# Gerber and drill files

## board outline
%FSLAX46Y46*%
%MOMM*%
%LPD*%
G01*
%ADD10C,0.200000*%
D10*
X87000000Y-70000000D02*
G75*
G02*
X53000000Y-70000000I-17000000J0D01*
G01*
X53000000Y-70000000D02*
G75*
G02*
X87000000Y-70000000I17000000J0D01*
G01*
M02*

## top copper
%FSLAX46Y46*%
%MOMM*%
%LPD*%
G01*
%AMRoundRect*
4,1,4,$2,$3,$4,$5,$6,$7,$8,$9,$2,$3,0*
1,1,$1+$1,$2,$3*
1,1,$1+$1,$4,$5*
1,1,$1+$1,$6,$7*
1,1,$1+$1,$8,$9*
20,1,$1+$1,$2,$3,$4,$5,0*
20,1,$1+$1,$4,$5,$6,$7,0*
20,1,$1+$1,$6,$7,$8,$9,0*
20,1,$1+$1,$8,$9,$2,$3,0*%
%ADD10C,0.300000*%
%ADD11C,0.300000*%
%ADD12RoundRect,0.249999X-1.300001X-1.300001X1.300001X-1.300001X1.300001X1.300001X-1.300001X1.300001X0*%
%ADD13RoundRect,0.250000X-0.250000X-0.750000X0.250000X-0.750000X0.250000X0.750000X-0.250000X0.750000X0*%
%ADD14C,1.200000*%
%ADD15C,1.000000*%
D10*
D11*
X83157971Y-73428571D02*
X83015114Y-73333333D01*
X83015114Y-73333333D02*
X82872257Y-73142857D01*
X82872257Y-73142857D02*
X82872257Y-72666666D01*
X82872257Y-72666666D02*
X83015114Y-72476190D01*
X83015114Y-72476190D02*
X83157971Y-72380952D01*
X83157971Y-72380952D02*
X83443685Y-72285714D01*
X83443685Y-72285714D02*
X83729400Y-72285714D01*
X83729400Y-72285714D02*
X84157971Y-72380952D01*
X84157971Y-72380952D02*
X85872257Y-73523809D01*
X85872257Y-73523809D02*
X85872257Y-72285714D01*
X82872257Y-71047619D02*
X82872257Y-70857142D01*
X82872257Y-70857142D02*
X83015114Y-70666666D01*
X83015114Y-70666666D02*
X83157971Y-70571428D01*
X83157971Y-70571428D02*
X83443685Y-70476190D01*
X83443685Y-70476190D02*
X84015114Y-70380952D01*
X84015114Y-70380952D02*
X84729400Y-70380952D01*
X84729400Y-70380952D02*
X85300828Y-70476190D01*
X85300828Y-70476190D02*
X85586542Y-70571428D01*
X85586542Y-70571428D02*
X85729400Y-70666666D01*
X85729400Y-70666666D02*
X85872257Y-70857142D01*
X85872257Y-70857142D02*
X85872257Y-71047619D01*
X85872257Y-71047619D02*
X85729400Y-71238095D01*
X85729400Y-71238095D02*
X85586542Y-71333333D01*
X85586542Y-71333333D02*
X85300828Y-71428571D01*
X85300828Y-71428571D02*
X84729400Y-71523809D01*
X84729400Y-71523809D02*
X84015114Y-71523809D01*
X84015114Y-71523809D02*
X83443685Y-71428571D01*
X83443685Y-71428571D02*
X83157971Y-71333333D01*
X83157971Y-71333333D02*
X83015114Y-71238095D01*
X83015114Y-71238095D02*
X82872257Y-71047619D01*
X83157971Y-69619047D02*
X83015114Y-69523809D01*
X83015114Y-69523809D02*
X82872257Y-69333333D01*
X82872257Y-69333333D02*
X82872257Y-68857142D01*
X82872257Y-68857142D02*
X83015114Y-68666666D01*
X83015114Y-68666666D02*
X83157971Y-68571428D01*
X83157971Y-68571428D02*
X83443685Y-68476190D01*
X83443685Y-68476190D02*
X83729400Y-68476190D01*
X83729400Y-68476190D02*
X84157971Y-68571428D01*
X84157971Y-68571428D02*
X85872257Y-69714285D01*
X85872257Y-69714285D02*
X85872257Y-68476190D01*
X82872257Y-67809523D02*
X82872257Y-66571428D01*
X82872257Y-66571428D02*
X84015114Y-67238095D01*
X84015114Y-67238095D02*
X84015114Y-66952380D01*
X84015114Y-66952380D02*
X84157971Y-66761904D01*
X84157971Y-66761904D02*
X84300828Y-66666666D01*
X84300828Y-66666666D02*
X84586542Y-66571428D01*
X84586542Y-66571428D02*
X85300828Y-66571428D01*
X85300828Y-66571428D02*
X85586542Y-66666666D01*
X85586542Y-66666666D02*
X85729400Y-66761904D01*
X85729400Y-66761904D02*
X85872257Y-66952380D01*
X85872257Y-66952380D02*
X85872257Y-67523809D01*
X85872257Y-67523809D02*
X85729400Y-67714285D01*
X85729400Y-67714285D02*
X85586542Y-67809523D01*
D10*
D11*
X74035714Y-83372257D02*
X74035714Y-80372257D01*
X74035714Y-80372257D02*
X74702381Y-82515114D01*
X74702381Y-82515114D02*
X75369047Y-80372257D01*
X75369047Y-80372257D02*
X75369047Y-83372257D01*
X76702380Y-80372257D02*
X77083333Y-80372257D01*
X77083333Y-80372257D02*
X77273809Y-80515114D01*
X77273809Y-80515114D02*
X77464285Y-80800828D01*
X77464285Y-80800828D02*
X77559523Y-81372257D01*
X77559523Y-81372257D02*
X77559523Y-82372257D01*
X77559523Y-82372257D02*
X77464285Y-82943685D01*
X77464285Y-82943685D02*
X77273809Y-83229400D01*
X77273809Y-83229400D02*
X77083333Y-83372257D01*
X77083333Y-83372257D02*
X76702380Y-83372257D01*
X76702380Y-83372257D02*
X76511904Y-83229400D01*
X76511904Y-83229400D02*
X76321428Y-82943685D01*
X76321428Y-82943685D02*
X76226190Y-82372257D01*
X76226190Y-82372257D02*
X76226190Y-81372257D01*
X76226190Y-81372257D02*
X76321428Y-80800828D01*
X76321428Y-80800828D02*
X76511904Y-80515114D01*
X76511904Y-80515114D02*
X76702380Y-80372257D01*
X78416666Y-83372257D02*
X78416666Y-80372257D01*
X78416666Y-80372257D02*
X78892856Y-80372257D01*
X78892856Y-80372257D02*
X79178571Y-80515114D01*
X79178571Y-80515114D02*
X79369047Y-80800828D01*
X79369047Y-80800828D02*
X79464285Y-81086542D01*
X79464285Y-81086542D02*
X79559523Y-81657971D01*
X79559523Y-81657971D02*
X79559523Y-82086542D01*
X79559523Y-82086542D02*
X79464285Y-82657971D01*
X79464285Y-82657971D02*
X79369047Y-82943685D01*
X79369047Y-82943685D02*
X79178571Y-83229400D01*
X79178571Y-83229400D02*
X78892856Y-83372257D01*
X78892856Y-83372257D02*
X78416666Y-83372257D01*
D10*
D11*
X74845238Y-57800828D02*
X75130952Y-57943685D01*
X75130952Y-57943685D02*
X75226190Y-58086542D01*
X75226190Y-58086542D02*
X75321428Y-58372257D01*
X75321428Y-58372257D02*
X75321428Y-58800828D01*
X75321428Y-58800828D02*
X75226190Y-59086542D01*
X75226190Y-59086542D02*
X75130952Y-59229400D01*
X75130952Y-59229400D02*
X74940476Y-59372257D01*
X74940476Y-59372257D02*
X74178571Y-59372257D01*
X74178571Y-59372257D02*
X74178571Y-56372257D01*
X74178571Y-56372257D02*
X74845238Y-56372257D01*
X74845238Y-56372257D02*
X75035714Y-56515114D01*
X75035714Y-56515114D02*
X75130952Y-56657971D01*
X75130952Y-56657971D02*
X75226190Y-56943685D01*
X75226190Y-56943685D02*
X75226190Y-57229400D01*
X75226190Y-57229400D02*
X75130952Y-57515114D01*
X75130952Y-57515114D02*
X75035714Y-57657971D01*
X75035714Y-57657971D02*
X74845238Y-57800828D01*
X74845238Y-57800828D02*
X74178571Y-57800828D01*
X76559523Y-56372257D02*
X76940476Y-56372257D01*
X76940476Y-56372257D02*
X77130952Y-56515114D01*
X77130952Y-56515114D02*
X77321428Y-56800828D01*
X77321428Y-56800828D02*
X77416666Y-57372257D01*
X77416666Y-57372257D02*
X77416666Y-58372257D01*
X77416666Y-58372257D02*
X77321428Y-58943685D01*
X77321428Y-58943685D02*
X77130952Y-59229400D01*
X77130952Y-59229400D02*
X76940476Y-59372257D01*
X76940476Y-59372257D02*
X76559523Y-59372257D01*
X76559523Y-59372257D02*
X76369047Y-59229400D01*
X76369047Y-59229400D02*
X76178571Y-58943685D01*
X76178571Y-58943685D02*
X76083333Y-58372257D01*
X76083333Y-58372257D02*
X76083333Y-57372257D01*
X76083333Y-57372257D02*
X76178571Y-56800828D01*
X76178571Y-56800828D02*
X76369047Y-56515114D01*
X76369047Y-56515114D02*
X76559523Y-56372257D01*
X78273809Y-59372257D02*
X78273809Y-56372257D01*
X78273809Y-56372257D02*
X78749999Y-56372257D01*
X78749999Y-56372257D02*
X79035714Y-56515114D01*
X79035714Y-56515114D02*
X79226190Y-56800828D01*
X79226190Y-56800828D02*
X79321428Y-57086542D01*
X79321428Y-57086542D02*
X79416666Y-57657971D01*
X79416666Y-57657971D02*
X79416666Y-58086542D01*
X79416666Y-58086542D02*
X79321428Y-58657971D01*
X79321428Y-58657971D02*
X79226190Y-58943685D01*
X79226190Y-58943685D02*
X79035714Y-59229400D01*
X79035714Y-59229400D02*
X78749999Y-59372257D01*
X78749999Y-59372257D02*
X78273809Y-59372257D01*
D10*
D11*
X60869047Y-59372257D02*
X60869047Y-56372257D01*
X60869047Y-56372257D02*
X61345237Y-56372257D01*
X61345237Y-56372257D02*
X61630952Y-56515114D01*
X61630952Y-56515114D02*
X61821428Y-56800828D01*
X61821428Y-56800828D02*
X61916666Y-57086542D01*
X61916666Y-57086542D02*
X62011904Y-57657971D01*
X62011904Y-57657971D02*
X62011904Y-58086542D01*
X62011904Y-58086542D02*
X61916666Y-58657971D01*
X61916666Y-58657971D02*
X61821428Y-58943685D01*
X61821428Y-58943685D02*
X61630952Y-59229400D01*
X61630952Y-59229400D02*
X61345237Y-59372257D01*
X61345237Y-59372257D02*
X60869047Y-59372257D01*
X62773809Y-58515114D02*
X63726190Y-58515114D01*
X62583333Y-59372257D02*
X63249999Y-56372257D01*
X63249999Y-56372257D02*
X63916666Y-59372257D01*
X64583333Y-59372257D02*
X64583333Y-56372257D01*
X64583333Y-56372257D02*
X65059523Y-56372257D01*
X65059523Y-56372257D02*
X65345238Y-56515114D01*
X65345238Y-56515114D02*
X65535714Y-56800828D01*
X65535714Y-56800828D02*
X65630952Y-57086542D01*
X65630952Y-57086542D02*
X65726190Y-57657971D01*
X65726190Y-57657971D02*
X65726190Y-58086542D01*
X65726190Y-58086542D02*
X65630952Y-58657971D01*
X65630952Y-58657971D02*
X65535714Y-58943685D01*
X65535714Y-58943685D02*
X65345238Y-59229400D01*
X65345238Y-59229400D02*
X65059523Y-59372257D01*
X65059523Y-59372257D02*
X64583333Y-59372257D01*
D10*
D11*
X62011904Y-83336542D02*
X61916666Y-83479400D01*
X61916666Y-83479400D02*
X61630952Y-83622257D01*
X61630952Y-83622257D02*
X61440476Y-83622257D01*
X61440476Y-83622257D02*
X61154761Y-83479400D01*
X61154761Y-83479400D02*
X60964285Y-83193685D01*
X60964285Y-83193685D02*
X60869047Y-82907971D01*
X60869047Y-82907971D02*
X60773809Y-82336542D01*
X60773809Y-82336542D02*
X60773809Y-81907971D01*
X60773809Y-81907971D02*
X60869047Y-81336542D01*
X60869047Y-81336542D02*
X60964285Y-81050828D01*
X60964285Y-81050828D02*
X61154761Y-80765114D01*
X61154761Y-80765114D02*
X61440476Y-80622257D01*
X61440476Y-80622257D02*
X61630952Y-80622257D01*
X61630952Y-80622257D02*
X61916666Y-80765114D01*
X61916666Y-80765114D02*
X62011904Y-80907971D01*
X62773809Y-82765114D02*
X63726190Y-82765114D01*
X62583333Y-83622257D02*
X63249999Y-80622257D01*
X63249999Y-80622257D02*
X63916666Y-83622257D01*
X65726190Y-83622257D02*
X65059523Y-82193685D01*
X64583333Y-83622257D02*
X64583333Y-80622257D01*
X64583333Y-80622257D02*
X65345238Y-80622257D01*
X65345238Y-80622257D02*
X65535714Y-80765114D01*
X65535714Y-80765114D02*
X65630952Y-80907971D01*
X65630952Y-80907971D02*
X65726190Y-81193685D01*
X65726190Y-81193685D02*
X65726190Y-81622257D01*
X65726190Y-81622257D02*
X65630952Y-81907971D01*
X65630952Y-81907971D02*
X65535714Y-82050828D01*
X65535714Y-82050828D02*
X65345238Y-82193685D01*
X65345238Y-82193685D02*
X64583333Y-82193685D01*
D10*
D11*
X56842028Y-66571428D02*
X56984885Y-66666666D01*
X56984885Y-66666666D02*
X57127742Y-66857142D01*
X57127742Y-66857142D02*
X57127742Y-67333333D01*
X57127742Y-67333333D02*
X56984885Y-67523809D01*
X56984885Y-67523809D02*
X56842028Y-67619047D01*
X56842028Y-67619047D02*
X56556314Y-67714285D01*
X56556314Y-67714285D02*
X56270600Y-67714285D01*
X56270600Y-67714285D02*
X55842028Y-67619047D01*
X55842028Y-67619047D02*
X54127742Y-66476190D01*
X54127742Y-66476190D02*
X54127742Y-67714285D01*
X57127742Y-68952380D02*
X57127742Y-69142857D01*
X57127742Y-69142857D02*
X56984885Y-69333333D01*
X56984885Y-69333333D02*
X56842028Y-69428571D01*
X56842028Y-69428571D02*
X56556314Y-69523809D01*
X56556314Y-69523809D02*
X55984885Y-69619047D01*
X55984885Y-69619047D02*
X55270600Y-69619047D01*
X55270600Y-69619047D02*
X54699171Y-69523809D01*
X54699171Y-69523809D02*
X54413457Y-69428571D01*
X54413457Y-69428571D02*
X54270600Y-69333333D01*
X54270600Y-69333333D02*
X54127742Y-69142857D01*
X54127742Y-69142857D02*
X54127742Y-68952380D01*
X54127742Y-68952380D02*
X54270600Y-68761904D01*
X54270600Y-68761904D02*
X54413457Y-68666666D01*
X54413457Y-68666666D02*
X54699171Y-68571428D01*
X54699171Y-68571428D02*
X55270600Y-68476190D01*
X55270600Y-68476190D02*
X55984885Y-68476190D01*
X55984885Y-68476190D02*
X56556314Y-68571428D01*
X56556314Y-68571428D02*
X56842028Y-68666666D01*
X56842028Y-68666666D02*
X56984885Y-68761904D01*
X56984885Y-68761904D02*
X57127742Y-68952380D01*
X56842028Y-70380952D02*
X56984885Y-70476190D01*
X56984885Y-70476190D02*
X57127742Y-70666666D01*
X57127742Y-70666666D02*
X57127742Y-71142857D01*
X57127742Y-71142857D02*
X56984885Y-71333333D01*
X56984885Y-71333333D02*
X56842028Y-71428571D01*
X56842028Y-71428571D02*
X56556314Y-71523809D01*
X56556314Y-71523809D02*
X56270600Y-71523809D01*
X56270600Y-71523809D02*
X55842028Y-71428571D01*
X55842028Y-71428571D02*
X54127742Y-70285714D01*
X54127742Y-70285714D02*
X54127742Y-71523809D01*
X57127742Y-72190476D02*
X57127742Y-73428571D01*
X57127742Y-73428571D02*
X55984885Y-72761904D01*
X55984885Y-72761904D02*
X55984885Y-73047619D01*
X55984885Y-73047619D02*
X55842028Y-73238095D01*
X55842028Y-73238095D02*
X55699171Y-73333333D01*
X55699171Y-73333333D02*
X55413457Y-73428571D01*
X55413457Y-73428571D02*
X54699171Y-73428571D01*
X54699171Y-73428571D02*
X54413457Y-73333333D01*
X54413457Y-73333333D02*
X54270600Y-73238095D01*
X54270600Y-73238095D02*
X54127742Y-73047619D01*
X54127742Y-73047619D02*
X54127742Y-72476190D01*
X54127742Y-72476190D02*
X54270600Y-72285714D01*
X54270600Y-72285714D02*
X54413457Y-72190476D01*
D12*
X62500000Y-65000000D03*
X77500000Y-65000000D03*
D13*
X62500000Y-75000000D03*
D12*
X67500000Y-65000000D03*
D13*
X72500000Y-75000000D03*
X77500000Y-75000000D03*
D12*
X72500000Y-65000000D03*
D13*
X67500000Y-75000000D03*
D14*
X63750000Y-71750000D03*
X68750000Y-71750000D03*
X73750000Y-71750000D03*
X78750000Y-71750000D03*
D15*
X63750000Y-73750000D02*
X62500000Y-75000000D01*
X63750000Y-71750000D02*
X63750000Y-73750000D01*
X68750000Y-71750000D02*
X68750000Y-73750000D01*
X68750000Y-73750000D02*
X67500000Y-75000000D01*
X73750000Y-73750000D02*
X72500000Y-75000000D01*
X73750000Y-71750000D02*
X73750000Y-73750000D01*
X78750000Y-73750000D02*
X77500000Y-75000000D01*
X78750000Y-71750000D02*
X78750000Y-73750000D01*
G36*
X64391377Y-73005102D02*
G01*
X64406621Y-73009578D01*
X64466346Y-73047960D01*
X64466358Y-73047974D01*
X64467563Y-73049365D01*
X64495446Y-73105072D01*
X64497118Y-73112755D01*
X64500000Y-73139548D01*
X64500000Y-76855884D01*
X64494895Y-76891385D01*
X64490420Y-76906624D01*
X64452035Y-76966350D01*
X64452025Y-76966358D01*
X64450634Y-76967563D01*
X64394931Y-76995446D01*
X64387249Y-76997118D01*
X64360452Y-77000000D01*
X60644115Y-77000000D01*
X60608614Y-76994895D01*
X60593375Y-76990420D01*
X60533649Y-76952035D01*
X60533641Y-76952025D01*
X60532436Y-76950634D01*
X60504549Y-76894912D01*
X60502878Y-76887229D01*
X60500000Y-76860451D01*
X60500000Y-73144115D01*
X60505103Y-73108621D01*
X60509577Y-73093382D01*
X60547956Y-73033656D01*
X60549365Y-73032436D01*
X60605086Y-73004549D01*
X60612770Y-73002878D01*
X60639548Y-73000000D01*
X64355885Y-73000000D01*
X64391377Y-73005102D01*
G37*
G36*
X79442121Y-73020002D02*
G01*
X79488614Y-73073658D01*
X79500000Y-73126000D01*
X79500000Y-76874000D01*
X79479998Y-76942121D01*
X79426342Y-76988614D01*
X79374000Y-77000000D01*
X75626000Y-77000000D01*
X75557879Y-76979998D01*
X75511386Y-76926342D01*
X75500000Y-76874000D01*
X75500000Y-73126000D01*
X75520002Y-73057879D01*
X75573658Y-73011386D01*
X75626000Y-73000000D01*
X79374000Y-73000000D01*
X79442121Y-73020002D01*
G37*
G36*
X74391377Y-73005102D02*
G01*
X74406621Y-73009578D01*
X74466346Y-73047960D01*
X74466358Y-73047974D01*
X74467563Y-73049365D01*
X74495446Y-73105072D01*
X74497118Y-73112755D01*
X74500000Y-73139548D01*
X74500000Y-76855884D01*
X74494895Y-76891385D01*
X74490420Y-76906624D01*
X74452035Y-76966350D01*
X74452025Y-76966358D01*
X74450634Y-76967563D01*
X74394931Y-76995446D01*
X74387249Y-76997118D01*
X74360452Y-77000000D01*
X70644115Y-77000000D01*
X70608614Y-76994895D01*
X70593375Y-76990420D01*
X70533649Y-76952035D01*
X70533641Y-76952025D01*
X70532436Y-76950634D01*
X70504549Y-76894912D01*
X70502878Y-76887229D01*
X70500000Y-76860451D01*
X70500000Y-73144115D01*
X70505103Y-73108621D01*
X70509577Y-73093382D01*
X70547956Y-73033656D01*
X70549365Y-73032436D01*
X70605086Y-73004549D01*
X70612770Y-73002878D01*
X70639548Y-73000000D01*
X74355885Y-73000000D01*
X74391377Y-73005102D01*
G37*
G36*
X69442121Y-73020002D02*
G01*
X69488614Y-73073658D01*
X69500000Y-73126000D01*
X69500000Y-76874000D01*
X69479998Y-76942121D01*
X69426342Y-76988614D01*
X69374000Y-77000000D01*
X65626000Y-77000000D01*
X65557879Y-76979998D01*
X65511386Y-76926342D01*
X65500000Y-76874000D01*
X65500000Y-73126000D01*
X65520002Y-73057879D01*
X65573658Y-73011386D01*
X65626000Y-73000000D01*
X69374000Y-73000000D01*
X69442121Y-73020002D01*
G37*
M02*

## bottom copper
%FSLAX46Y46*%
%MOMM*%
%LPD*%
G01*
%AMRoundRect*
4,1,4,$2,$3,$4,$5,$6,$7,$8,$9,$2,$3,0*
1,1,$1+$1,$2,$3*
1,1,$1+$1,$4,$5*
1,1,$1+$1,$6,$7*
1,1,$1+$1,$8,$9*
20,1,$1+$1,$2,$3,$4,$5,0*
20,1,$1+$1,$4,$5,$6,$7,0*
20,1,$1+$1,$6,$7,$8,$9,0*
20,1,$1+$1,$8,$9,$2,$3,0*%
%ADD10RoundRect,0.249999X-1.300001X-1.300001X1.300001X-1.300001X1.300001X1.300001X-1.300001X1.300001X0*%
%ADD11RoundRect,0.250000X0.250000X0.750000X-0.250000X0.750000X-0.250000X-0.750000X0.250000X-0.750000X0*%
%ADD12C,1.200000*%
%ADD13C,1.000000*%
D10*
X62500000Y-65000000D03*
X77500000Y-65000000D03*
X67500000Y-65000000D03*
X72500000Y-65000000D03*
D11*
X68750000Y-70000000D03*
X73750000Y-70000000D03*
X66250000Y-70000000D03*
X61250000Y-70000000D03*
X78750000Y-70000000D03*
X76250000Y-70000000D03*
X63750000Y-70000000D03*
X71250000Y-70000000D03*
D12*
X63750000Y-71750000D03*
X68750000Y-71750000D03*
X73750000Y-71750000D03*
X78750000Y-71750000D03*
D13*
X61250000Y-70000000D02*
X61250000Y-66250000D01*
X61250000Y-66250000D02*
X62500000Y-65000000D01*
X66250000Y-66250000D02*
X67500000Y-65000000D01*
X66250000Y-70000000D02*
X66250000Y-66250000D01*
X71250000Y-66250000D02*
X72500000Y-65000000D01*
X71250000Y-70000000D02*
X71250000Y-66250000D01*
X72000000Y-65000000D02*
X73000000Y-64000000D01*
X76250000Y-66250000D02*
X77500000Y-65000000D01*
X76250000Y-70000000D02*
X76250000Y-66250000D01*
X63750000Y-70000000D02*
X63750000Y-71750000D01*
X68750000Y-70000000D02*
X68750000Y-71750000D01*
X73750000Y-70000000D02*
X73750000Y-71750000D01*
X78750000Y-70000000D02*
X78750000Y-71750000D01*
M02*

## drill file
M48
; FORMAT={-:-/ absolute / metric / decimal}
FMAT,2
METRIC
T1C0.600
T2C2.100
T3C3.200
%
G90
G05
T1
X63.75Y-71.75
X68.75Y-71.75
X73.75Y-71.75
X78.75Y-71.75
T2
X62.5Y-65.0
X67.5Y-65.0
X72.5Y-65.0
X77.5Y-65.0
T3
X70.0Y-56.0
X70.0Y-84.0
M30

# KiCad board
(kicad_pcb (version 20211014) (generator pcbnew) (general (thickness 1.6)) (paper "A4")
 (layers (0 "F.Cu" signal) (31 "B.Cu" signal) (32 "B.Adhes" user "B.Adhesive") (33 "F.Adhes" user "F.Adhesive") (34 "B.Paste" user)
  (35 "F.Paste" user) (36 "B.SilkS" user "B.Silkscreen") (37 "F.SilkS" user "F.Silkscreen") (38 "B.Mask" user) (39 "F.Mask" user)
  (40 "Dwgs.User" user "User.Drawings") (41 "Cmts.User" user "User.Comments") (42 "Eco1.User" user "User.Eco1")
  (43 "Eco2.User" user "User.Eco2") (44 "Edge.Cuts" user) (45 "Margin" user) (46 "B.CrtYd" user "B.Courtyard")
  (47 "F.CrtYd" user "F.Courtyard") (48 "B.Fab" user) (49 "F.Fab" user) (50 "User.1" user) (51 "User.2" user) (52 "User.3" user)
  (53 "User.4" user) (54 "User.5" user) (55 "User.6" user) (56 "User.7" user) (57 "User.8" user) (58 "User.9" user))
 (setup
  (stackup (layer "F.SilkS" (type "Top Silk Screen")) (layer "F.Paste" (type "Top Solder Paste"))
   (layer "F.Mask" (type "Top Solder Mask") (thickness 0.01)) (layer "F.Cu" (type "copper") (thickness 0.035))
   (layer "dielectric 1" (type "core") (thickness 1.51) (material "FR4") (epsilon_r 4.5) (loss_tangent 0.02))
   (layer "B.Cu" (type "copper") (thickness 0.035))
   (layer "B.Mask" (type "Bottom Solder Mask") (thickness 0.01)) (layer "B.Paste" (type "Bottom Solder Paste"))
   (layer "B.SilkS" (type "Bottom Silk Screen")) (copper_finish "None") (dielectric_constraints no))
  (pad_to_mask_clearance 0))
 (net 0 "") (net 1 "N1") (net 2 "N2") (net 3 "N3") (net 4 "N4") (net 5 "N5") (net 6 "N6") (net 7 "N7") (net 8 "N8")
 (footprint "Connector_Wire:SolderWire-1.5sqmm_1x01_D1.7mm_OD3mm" (layer "F.Cu") (at 62.5 65)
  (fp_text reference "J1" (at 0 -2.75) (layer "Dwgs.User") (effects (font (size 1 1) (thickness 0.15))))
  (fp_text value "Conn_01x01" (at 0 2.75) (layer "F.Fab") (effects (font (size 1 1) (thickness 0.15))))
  (pad "1" thru_hole roundrect (at 0 0) (size 3.1 3.1) (drill 2.1) (layers *.Cu *.Mask) (roundrect_rratio 0.08064483871) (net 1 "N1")))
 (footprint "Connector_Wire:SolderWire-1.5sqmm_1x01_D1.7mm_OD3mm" (layer "F.Cu") (at 77.5 65)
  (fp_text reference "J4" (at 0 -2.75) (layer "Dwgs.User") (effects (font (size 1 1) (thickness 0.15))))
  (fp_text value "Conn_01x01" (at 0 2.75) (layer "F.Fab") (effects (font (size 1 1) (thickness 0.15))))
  (pad "1" thru_hole roundrect (at 0 0) (size 3.1 3.1) (drill 2.1) (layers *.Cu *.Mask) (roundrect_rratio 0.08064483871) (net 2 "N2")))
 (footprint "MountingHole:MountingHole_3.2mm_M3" (layer "F.Cu") (at 70 84)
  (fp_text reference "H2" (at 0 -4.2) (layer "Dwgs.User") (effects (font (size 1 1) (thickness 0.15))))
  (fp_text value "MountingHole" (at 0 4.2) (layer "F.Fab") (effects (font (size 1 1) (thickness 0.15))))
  (pad "" np_thru_hole circle (at 0 0) (size 3.2 3.2) (drill 3.2) (layers *.Cu *.Mask)))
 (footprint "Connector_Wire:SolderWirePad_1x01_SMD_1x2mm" (layer "F.Cu") (at 62.5 75)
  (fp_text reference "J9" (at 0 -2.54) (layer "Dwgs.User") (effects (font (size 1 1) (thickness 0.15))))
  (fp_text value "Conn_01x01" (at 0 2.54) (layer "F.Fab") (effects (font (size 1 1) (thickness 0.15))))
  (pad "1" smd roundrect (at 0 0) (size 1 2) (layers "F.Cu" "F.Paste" "F.Mask") (roundrect_rratio 0.25) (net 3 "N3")))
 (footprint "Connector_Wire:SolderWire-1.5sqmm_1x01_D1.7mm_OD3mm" (layer "F.Cu") (at 67.5 65)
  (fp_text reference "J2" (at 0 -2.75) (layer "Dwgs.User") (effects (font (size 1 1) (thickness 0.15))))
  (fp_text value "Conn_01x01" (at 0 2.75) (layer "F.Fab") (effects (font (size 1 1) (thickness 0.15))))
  (pad "1" thru_hole roundrect (at 0 0) (size 3.1 3.1) (drill 2.1) (layers *.Cu *.Mask) (roundrect_rratio 0.08064483871) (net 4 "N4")))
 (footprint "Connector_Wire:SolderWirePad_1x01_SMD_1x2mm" (layer "F.Cu") (at 72.5 75)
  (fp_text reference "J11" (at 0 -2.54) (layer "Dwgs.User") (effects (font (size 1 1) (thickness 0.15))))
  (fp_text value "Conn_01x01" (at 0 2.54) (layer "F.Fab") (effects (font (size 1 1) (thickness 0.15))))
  (pad "1" smd roundrect (at 0 0) (size 1 2) (layers "F.Cu" "F.Paste" "F.Mask") (roundrect_rratio 0.25) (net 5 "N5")))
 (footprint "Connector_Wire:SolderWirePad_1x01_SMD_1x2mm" (layer "F.Cu") (at 77.5 75)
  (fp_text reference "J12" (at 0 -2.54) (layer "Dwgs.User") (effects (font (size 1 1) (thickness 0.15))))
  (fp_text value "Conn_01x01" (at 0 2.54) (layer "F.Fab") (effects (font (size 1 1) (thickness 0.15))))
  (pad "1" smd roundrect (at 0 0) (size 1 2) (layers "F.Cu" "F.Paste" "F.Mask") (roundrect_rratio 0.25) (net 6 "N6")))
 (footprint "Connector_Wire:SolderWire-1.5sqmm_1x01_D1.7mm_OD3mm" (layer "F.Cu") (at 72.5 65)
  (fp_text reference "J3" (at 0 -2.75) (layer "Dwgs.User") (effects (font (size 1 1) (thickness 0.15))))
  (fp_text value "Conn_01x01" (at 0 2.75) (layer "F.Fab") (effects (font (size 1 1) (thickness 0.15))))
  (pad "1" thru_hole roundrect (at 0 0) (size 3.1 3.1) (drill 2.1) (layers *.Cu *.Mask) (roundrect_rratio 0.08064483871) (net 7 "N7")))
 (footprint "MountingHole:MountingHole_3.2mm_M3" (layer "F.Cu") (at 70 56)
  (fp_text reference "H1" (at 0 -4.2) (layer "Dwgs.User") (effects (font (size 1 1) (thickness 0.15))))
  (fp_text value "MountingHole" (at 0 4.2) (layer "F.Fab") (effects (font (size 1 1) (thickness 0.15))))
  (pad "" np_thru_hole circle (at 0 0) (size 3.2 3.2) (drill 3.2) (layers *.Cu *.Mask)))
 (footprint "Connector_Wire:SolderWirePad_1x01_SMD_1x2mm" (layer "F.Cu") (at 67.5 75)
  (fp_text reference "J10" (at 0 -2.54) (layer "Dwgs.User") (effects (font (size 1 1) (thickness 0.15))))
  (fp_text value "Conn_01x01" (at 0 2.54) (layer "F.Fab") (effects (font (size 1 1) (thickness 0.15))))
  (pad "1" smd roundrect (at 0 0) (size 1 2) (layers "F.Cu" "F.Paste" "F.Mask") (roundrect_rratio 0.25) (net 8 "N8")))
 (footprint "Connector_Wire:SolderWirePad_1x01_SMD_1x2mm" (layer "B.Cu") (at 68.75 70 180)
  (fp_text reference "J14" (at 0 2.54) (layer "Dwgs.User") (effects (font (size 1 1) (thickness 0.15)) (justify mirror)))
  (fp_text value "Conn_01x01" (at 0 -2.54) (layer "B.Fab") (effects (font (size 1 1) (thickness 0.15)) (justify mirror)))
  (pad "1" smd roundrect (at 0 0 180) (size 1 2) (layers "B.Cu" "B.Paste" "B.Mask") (roundrect_rratio 0.25) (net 8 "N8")))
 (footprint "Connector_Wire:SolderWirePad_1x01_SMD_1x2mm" (layer "B.Cu") (at 73.75 70 180)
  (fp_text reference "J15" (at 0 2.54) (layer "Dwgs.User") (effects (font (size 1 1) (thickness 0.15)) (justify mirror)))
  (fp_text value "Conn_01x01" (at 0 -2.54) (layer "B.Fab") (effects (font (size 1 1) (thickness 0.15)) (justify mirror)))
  (pad "1" smd roundrect (at 0 0 180) (size 1 2) (layers "B.Cu" "B.Paste" "B.Mask") (roundrect_rratio 0.25) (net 5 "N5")))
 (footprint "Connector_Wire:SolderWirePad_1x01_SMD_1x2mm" (layer "B.Cu") (at 66.25 70 180)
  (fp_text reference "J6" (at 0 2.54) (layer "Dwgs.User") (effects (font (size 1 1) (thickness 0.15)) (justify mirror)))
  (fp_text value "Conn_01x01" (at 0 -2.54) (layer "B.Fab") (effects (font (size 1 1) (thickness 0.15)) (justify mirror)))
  (pad "1" smd roundrect (at 0 0 180) (size 1 2) (layers "B.Cu" "B.Paste" "B.Mask") (roundrect_rratio 0.25) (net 4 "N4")))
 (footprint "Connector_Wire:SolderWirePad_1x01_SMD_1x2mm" (layer "B.Cu") (at 61.25 70 180)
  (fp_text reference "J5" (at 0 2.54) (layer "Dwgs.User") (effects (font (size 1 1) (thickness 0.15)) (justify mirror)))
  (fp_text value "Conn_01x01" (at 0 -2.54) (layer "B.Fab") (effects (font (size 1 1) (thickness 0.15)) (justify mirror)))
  (pad "1" smd roundrect (at 0 0 180) (size 1 2) (layers "B.Cu" "B.Paste" "B.Mask") (roundrect_rratio 0.25) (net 1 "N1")))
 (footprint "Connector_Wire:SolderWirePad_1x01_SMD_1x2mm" (layer "B.Cu") (at 78.75 70 180)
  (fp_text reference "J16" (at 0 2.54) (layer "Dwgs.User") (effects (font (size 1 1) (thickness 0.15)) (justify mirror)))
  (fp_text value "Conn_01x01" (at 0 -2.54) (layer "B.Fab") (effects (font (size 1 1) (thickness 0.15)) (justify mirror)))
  (pad "1" smd roundrect (at 0 0 180) (size 1 2) (layers "B.Cu" "B.Paste" "B.Mask") (roundrect_rratio 0.25) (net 6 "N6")))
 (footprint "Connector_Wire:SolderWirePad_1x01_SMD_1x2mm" (layer "B.Cu") (at 76.25 70 180)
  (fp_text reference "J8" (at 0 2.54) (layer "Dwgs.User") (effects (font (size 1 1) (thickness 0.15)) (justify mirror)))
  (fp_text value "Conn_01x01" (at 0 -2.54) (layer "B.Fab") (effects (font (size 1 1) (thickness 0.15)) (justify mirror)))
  (pad "1" smd roundrect (at 0 0 180) (size 1 2) (layers "B.Cu" "B.Paste" "B.Mask") (roundrect_rratio 0.25) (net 2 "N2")))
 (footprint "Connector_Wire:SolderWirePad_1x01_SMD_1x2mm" (layer "B.Cu") (at 63.75 70 180)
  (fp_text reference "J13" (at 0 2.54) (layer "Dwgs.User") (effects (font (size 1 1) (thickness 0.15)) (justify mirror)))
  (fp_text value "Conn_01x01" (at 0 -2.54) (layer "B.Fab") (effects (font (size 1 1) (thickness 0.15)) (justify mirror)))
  (pad "1" smd roundrect (at 0 0 180) (size 1 2) (layers "B.Cu" "B.Paste" "B.Mask") (roundrect_rratio 0.25) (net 3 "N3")))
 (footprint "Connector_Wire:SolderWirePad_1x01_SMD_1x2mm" (layer "B.Cu") (at 71.25 70 180)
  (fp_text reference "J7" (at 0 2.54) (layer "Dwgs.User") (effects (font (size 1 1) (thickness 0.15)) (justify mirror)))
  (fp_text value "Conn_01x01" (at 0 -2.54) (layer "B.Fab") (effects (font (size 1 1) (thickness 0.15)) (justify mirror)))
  (pad "1" smd roundrect (at 0 0 180) (size 1 2) (layers "B.Cu" "B.Paste" "B.Mask") (roundrect_rratio 0.25) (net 7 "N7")))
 (gr_circle (center 70 70) (end 87 70) (layer "Edge.Cuts") (width 0.2) (fill none))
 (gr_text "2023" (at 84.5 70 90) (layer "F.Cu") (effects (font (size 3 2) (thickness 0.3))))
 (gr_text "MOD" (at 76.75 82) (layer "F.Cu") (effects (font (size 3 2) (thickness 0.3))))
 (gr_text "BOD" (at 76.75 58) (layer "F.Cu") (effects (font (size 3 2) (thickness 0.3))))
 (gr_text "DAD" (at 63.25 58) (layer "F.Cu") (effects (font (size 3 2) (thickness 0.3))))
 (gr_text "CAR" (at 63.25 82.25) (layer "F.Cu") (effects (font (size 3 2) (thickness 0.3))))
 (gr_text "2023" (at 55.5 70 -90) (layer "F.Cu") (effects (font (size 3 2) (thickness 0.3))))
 (segment (start 61.25 70) (end 61.25 66.25) (width 1) (layer "B.Cu") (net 1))
 (segment (start 61.25 66.25) (end 62.5 65) (width 1) (layer "B.Cu") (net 1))
 (segment (start 66.25 66.25) (end 67.5 65) (width 1) (layer "B.Cu") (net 4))
 (segment (start 66.25 70) (end 66.25 66.25) (width 1) (layer "B.Cu") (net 4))
 (segment (start 71.25 66.25) (end 72.5 65) (width 1) (layer "B.Cu") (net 7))
 (segment (start 71.25 70) (end 71.25 66.25) (width 1) (layer "B.Cu") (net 7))
 (segment (start 72 65) (end 73 64) (width 1) (layer "B.Cu") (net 7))
 (segment (start 76.25 66.25) (end 77.5 65) (width 1) (layer "B.Cu") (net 2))
 (segment (start 76.25 70) (end 76.25 66.25) (width 1) (layer "B.Cu") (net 2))
 (segment (start 63.75 73.75) (end 62.5 75) (width 1) (layer "F.Cu") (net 3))
 (segment (start 63.75 71.75) (end 63.75 73.75) (width 1) (layer "F.Cu") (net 3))
 (via (at 63.75 71.75) (size 1.2) (drill 0.6) (layers "F.Cu" "B.Cu") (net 3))
 (segment (start 63.75 70) (end 63.75 71.75) (width 1) (layer "B.Cu") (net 3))
 (segment (start 68.75 71.75) (end 68.75 73.75) (width 1) (layer "F.Cu") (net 8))
 (segment (start 68.75 73.75) (end 67.5 75) (width 1) (layer "F.Cu") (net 8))
 (via (at 68.75 71.75) (size 1.2) (drill 0.6) (layers "F.Cu" "B.Cu") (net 8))
 (segment (start 68.75 70) (end 68.75 71.75) (width 1) (layer "B.Cu") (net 8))
 (segment (start 73.75 73.75) (end 72.5 75) (width 1) (layer "F.Cu") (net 5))
 (segment (start 73.75 71.75) (end 73.75 73.75) (width 1) (layer "F.Cu") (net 5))
 (via (at 73.75 71.75) (size 1.2) (drill 0.6) (layers "F.Cu" "B.Cu") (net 5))
 (segment (start 73.75 70) (end 73.75 71.75) (width 1) (layer "B.Cu") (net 5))
 (segment (start 78.75 73.75) (end 77.5 75) (width 1) (layer "F.Cu") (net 6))
 (segment (start 78.75 71.75) (end 78.75 73.75) (width 1) (layer "F.Cu") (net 6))
 (via (at 78.75 71.75) (size 1.2) (drill 0.6) (layers "F.Cu" "B.Cu") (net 6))
 (segment (start 78.75 70) (end 78.75 71.75) (width 1) (layer "B.Cu") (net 6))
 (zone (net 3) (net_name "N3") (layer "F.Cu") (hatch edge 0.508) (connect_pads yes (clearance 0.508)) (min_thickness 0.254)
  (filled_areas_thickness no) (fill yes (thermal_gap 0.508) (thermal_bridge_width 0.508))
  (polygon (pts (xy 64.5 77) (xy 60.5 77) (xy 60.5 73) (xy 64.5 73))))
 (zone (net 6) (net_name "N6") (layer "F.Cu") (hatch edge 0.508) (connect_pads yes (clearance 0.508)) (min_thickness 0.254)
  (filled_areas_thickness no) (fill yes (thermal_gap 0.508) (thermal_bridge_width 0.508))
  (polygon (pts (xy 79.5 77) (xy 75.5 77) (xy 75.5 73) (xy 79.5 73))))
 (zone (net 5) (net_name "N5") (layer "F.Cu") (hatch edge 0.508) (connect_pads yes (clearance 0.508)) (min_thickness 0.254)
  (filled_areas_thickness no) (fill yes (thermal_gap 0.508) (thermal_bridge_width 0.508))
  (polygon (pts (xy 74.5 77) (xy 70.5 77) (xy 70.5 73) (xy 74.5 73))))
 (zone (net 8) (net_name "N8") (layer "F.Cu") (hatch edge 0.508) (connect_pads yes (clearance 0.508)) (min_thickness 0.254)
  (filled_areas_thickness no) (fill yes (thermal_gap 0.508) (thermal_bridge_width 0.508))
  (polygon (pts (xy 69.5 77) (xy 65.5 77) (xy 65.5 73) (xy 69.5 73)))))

